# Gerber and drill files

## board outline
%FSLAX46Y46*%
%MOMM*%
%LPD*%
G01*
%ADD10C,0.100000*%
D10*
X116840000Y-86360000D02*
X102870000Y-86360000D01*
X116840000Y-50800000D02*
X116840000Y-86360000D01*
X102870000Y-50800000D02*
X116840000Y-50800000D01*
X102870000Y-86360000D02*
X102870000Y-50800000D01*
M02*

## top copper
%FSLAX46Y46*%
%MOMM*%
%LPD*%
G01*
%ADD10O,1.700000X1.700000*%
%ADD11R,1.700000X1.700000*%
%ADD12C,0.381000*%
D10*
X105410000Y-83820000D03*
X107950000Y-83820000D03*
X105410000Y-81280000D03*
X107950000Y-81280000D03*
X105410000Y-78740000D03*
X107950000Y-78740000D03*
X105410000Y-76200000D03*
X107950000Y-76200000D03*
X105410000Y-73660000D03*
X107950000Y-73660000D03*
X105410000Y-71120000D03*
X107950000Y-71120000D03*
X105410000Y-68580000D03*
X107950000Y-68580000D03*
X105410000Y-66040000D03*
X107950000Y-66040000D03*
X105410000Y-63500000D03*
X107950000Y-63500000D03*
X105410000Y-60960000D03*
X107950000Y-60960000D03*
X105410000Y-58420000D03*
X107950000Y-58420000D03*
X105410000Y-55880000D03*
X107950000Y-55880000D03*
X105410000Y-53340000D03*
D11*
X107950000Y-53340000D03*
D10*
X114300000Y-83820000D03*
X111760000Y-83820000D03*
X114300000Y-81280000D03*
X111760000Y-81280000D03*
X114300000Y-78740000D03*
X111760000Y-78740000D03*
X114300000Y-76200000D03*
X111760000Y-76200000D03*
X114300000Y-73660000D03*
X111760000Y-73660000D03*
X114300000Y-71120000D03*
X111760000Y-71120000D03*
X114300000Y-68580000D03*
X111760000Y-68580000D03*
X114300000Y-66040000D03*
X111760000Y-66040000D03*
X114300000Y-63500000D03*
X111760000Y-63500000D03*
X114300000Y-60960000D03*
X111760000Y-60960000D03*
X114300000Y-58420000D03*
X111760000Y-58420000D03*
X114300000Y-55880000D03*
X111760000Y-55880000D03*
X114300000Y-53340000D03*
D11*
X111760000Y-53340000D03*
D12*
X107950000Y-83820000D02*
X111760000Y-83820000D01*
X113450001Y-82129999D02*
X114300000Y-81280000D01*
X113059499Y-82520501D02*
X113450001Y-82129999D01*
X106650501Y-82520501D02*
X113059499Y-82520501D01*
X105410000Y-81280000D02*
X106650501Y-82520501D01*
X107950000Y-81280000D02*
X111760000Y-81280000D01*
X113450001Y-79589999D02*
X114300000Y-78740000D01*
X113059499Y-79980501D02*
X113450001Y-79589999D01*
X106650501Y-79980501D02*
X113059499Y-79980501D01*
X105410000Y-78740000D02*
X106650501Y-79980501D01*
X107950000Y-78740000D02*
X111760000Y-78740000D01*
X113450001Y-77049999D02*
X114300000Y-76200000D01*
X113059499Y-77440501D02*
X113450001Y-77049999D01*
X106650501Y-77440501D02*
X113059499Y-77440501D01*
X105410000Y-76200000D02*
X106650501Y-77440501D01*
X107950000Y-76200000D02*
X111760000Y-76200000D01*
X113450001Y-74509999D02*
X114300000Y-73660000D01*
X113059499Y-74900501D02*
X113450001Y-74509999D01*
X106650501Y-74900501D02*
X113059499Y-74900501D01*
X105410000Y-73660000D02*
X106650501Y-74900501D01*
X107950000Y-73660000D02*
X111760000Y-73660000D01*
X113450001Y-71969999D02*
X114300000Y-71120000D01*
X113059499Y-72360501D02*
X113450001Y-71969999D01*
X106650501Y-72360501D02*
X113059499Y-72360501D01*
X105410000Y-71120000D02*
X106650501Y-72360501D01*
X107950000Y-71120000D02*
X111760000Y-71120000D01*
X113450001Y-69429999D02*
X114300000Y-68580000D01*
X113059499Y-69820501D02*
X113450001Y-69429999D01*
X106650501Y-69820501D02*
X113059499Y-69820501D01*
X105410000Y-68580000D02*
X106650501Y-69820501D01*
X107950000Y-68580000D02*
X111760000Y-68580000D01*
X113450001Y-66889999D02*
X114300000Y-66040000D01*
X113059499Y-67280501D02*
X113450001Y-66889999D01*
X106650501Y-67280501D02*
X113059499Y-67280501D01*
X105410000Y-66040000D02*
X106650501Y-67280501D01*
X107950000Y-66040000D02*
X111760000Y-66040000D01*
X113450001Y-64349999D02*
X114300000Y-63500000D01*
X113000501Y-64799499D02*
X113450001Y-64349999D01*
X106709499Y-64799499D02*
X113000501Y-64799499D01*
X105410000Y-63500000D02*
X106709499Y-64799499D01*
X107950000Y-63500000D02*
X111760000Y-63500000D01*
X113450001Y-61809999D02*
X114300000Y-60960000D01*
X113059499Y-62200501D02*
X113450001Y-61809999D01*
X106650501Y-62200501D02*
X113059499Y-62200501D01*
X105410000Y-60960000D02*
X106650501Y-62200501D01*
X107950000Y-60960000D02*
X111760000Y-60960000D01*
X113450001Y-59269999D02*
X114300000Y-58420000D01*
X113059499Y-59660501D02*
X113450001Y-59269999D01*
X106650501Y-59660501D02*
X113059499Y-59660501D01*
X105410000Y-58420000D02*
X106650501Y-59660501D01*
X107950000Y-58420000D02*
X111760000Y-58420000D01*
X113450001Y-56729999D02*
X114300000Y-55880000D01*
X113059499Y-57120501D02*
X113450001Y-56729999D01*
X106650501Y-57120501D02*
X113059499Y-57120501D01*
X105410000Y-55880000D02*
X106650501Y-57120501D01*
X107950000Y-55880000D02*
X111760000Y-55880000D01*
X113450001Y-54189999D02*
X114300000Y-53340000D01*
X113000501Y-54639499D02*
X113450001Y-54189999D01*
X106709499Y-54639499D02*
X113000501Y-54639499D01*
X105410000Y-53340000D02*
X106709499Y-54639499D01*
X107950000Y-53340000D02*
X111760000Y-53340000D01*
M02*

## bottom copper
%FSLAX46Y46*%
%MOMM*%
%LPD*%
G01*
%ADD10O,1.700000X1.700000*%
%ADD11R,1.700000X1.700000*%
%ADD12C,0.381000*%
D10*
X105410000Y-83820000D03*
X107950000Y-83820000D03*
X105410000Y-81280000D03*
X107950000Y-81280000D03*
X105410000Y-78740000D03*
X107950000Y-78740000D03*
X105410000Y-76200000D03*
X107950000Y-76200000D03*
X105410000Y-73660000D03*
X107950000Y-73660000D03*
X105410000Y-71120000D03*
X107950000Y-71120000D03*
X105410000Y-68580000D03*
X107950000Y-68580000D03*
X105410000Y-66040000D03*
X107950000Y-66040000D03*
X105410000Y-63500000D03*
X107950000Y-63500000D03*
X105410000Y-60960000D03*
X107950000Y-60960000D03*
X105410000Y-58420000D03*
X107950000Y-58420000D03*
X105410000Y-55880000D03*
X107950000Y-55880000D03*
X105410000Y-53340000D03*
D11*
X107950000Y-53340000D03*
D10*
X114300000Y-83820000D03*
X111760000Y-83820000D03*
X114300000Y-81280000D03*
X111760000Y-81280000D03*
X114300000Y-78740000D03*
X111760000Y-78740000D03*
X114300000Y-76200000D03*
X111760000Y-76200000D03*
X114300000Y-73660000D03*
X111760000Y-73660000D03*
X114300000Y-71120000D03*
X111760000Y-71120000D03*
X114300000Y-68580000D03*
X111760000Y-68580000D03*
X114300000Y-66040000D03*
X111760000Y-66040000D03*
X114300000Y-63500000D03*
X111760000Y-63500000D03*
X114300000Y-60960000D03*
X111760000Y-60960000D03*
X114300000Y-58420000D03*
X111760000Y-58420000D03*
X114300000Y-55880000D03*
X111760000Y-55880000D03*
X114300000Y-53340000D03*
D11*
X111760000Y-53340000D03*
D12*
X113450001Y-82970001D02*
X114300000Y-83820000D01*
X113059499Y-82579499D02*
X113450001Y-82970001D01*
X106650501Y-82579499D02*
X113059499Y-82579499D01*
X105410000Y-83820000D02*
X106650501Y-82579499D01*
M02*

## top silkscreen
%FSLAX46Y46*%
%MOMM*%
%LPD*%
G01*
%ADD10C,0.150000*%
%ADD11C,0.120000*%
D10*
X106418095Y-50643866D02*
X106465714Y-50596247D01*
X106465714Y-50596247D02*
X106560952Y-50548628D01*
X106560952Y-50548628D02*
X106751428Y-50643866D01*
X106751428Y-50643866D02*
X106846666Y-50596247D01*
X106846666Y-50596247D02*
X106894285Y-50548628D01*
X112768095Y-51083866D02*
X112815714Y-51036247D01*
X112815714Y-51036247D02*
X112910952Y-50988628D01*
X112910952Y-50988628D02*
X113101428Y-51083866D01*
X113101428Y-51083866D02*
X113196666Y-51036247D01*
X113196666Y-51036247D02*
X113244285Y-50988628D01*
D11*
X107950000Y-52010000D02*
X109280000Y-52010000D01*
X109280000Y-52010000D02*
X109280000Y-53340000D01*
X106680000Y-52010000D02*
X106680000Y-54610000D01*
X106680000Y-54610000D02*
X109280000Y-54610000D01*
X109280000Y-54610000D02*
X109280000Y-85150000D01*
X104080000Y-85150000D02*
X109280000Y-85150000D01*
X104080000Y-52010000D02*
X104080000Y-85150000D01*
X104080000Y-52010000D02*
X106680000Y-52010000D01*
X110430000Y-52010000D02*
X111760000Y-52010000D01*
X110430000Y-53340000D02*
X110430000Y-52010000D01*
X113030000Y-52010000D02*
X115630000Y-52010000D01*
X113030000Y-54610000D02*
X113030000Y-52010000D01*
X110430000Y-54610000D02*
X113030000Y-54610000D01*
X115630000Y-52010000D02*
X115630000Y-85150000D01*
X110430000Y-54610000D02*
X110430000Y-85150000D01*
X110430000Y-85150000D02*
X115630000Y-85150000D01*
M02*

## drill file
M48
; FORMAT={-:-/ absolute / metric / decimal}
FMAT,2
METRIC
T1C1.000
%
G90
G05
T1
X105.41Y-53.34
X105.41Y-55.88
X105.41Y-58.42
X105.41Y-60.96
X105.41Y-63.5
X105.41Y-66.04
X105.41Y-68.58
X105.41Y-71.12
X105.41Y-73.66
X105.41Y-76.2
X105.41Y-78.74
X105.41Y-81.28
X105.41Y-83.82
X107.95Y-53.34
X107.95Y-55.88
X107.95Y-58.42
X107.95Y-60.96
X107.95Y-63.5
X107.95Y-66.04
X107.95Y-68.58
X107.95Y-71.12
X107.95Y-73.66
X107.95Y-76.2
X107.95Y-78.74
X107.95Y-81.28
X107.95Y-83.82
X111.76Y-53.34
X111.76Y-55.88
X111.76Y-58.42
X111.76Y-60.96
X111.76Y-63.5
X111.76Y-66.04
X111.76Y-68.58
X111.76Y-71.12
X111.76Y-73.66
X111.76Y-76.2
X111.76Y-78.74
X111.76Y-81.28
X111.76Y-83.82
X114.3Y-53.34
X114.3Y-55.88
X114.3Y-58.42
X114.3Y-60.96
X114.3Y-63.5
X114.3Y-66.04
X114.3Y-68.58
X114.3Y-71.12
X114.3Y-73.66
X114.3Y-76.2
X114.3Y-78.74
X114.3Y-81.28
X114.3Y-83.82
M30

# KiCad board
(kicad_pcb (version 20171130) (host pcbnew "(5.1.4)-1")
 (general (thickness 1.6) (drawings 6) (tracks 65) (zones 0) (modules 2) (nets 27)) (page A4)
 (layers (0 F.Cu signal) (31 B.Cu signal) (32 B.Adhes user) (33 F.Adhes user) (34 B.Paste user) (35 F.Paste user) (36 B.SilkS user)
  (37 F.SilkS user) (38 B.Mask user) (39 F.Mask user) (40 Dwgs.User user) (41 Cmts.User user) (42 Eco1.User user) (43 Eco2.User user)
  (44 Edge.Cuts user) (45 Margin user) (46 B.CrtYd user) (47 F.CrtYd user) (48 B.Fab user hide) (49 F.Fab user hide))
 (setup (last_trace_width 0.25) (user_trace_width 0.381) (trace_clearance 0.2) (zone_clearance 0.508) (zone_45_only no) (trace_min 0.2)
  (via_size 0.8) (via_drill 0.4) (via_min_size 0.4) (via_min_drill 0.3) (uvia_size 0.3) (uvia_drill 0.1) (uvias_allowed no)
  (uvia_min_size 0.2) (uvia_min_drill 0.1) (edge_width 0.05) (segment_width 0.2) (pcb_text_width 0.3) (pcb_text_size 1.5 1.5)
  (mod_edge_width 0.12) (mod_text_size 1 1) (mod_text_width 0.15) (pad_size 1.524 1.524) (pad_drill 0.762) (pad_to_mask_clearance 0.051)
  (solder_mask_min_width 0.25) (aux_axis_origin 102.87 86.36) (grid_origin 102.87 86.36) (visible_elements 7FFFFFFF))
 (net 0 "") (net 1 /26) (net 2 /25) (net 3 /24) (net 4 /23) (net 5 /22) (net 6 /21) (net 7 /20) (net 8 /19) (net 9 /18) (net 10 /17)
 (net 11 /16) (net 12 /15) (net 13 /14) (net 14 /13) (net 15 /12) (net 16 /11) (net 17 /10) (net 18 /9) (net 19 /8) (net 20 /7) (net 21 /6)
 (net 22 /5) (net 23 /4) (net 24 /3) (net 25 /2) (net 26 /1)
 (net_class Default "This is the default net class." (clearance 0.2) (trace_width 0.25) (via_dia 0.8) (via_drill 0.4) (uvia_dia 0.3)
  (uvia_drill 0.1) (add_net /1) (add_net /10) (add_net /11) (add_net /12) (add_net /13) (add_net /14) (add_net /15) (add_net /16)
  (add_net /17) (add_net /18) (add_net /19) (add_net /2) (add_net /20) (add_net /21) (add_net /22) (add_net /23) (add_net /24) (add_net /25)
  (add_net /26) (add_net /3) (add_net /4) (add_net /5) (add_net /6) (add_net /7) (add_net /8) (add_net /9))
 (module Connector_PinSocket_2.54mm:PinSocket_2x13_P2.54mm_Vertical (layer F.Cu) (at 107.95 53.34)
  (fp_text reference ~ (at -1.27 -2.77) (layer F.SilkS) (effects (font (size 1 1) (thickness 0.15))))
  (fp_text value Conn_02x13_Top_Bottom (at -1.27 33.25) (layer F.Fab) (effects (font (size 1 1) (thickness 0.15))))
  (fp_line (start 0 -1.33) (end 1.33 -1.33) (layer F.SilkS) (width 0.12))
  (fp_line (start 1.33 -1.33) (end 1.33 0) (layer F.SilkS) (width 0.12))
  (fp_line (start -1.27 -1.33) (end -1.27 1.27) (layer F.SilkS) (width 0.12))
  (fp_line (start -1.27 1.27) (end 1.33 1.27) (layer F.SilkS) (width 0.12))
  (fp_line (start 1.33 1.27) (end 1.33 31.81) (layer F.SilkS) (width 0.12))
  (fp_line (start -3.87 31.81) (end 1.33 31.81) (layer F.SilkS) (width 0.12))
  (fp_line (start -3.87 -1.33) (end -3.87 31.81) (layer F.SilkS) (width 0.12))
  (fp_line (start -3.87 -1.33) (end -1.27 -1.33) (layer F.SilkS) (width 0.12))
  (pad 26 thru_hole oval (at -2.54 30.48) (size 1.7 1.7) (drill 1) (layers *.Cu *.Mask) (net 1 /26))
  (pad 25 thru_hole oval (at 0 30.48) (size 1.7 1.7) (drill 1) (layers *.Cu *.Mask) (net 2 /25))
  (pad 24 thru_hole oval (at -2.54 27.94) (size 1.7 1.7) (drill 1) (layers *.Cu *.Mask) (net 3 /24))
  (pad 23 thru_hole oval (at 0 27.94) (size 1.7 1.7) (drill 1) (layers *.Cu *.Mask) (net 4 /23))
  (pad 22 thru_hole oval (at -2.54 25.4) (size 1.7 1.7) (drill 1) (layers *.Cu *.Mask) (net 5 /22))
  (pad 21 thru_hole oval (at 0 25.4) (size 1.7 1.7) (drill 1) (layers *.Cu *.Mask) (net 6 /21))
  (pad 20 thru_hole oval (at -2.54 22.86) (size 1.7 1.7) (drill 1) (layers *.Cu *.Mask) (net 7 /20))
  (pad 19 thru_hole oval (at 0 22.86) (size 1.7 1.7) (drill 1) (layers *.Cu *.Mask) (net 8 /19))
  (pad 18 thru_hole oval (at -2.54 20.32) (size 1.7 1.7) (drill 1) (layers *.Cu *.Mask) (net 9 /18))
  (pad 17 thru_hole oval (at 0 20.32) (size 1.7 1.7) (drill 1) (layers *.Cu *.Mask) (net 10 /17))
  (pad 16 thru_hole oval (at -2.54 17.78) (size 1.7 1.7) (drill 1) (layers *.Cu *.Mask) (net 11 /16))
  (pad 15 thru_hole oval (at 0 17.78) (size 1.7 1.7) (drill 1) (layers *.Cu *.Mask) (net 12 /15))
  (pad 14 thru_hole oval (at -2.54 15.24) (size 1.7 1.7) (drill 1) (layers *.Cu *.Mask) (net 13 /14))
  (pad 13 thru_hole oval (at 0 15.24) (size 1.7 1.7) (drill 1) (layers *.Cu *.Mask) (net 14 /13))
  (pad 12 thru_hole oval (at -2.54 12.7) (size 1.7 1.7) (drill 1) (layers *.Cu *.Mask) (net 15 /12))
  (pad 11 thru_hole oval (at 0 12.7) (size 1.7 1.7) (drill 1) (layers *.Cu *.Mask) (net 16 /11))
  (pad 10 thru_hole oval (at -2.54 10.16) (size 1.7 1.7) (drill 1) (layers *.Cu *.Mask) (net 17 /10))
  (pad 9 thru_hole oval (at 0 10.16) (size 1.7 1.7) (drill 1) (layers *.Cu *.Mask) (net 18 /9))
  (pad 8 thru_hole oval (at -2.54 7.62) (size 1.7 1.7) (drill 1) (layers *.Cu *.Mask) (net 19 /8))
  (pad 7 thru_hole oval (at 0 7.62) (size 1.7 1.7) (drill 1) (layers *.Cu *.Mask) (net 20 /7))
  (pad 6 thru_hole oval (at -2.54 5.08) (size 1.7 1.7) (drill 1) (layers *.Cu *.Mask) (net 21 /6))
  (pad 5 thru_hole oval (at 0 5.08) (size 1.7 1.7) (drill 1) (layers *.Cu *.Mask) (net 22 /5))
  (pad 4 thru_hole oval (at -2.54 2.54) (size 1.7 1.7) (drill 1) (layers *.Cu *.Mask) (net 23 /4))
  (pad 3 thru_hole oval (at 0 2.54) (size 1.7 1.7) (drill 1) (layers *.Cu *.Mask) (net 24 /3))
  (pad 2 thru_hole oval (at -2.54 0) (size 1.7 1.7) (drill 1) (layers *.Cu *.Mask) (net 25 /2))
  (pad 1 thru_hole rect (at 0 0) (size 1.7 1.7) (drill 1) (layers *.Cu *.Mask) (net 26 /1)))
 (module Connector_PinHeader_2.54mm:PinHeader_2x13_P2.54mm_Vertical (layer F.Cu) (at 111.76 53.34)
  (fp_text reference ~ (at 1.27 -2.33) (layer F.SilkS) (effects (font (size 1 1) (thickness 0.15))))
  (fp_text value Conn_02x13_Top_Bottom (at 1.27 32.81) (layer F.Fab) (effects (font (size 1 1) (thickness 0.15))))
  (fp_line (start -1.33 -1.33) (end 0 -1.33) (layer F.SilkS) (width 0.12))
  (fp_line (start -1.33 0) (end -1.33 -1.33) (layer F.SilkS) (width 0.12))
  (fp_line (start 1.27 -1.33) (end 3.87 -1.33) (layer F.SilkS) (width 0.12))
  (fp_line (start 1.27 1.27) (end 1.27 -1.33) (layer F.SilkS) (width 0.12))
  (fp_line (start -1.33 1.27) (end 1.27 1.27) (layer F.SilkS) (width 0.12))
  (fp_line (start 3.87 -1.33) (end 3.87 31.81) (layer F.SilkS) (width 0.12))
  (fp_line (start -1.33 1.27) (end -1.33 31.81) (layer F.SilkS) (width 0.12))
  (fp_line (start -1.33 31.81) (end 3.87 31.81) (layer F.SilkS) (width 0.12))
  (pad 26 thru_hole oval (at 2.54 30.48) (size 1.7 1.7) (drill 1) (layers *.Cu *.Mask) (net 1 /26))
  (pad 25 thru_hole oval (at 0 30.48) (size 1.7 1.7) (drill 1) (layers *.Cu *.Mask) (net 2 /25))
  (pad 24 thru_hole oval (at 2.54 27.94) (size 1.7 1.7) (drill 1) (layers *.Cu *.Mask) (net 3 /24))
  (pad 23 thru_hole oval (at 0 27.94) (size 1.7 1.7) (drill 1) (layers *.Cu *.Mask) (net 4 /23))
  (pad 22 thru_hole oval (at 2.54 25.4) (size 1.7 1.7) (drill 1) (layers *.Cu *.Mask) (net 5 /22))
  (pad 21 thru_hole oval (at 0 25.4) (size 1.7 1.7) (drill 1) (layers *.Cu *.Mask) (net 6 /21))
  (pad 20 thru_hole oval (at 2.54 22.86) (size 1.7 1.7) (drill 1) (layers *.Cu *.Mask) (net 7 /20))
  (pad 19 thru_hole oval (at 0 22.86) (size 1.7 1.7) (drill 1) (layers *.Cu *.Mask) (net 8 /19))
  (pad 18 thru_hole oval (at 2.54 20.32) (size 1.7 1.7) (drill 1) (layers *.Cu *.Mask) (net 9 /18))
  (pad 17 thru_hole oval (at 0 20.32) (size 1.7 1.7) (drill 1) (layers *.Cu *.Mask) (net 10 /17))
  (pad 16 thru_hole oval (at 2.54 17.78) (size 1.7 1.7) (drill 1) (layers *.Cu *.Mask) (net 11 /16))
  (pad 15 thru_hole oval (at 0 17.78) (size 1.7 1.7) (drill 1) (layers *.Cu *.Mask) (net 12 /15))
  (pad 14 thru_hole oval (at 2.54 15.24) (size 1.7 1.7) (drill 1) (layers *.Cu *.Mask) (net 13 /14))
  (pad 13 thru_hole oval (at 0 15.24) (size 1.7 1.7) (drill 1) (layers *.Cu *.Mask) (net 14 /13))
  (pad 12 thru_hole oval (at 2.54 12.7) (size 1.7 1.7) (drill 1) (layers *.Cu *.Mask) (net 15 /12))
  (pad 11 thru_hole oval (at 0 12.7) (size 1.7 1.7) (drill 1) (layers *.Cu *.Mask) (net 16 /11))
  (pad 10 thru_hole oval (at 2.54 10.16) (size 1.7 1.7) (drill 1) (layers *.Cu *.Mask) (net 17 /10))
  (pad 9 thru_hole oval (at 0 10.16) (size 1.7 1.7) (drill 1) (layers *.Cu *.Mask) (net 18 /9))
  (pad 8 thru_hole oval (at 2.54 7.62) (size 1.7 1.7) (drill 1) (layers *.Cu *.Mask) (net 19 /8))
  (pad 7 thru_hole oval (at 0 7.62) (size 1.7 1.7) (drill 1) (layers *.Cu *.Mask) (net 20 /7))
  (pad 6 thru_hole oval (at 2.54 5.08) (size 1.7 1.7) (drill 1) (layers *.Cu *.Mask) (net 21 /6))
  (pad 5 thru_hole oval (at 0 5.08) (size 1.7 1.7) (drill 1) (layers *.Cu *.Mask) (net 22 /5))
  (pad 4 thru_hole oval (at 2.54 2.54) (size 1.7 1.7) (drill 1) (layers *.Cu *.Mask) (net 23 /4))
  (pad 3 thru_hole oval (at 0 2.54) (size 1.7 1.7) (drill 1) (layers *.Cu *.Mask) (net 24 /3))
  (pad 2 thru_hole oval (at 2.54 0) (size 1.7 1.7) (drill 1) (layers *.Cu *.Mask) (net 25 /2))
  (pad 1 thru_hole rect (at 0 0) (size 1.7 1.7) (drill 1) (layers *.Cu *.Mask) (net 26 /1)))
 (gr_line (start 116.84 86.36) (end 102.87 86.36) (layer Edge.Cuts) (width 0.1))
 (gr_line (start 116.84 50.8) (end 116.84 86.36) (layer Edge.Cuts) (width 0.1))
 (gr_line (start 102.87 50.8) (end 116.84 50.8) (layer Edge.Cuts) (width 0.1))
 (gr_line (start 102.87 86.36) (end 102.87 50.8) (layer Edge.Cuts) (width 0.1))
 (segment (start 113.450001 82.970001) (end 114.3 83.82) (width 0.381) (layer B.Cu) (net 1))
 (segment (start 113.059499 82.579499) (end 113.450001 82.970001) (width 0.381) (layer B.Cu) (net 1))
 (segment (start 106.650501 82.579499) (end 113.059499 82.579499) (width 0.381) (layer B.Cu) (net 1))
 (segment (start 105.41 83.82) (end 106.650501 82.579499) (width 0.381) (layer B.Cu) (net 1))
 (segment (start 107.95 83.82) (end 111.76 83.82) (width 0.381) (layer F.Cu) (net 2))
 (segment (start 113.450001 82.129999) (end 114.3 81.28) (width 0.381) (layer F.Cu) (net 3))
 (segment (start 113.059499 82.520501) (end 113.450001 82.129999) (width 0.381) (layer F.Cu) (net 3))
 (segment (start 106.650501 82.520501) (end 113.059499 82.520501) (width 0.381) (layer F.Cu) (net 3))
 (segment (start 105.41 81.28) (end 106.650501 82.520501) (width 0.381) (layer F.Cu) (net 3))
 (segment (start 107.95 81.28) (end 111.76 81.28) (width 0.381) (layer F.Cu) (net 4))
 (segment (start 113.450001 79.589999) (end 114.3 78.74) (width 0.381) (layer F.Cu) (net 5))
 (segment (start 113.059499 79.980501) (end 113.450001 79.589999) (width 0.381) (layer F.Cu) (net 5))
 (segment (start 106.650501 79.980501) (end 113.059499 79.980501) (width 0.381) (layer F.Cu) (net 5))
 (segment (start 105.41 78.74) (end 106.650501 79.980501) (width 0.381) (layer F.Cu) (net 5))
 (segment (start 107.95 78.74) (end 111.76 78.74) (width 0.381) (layer F.Cu) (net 6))
 (segment (start 113.450001 77.049999) (end 114.3 76.2) (width 0.381) (layer F.Cu) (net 7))
 (segment (start 113.059499 77.440501) (end 113.450001 77.049999) (width 0.381) (layer F.Cu) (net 7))
 (segment (start 106.650501 77.440501) (end 113.059499 77.440501) (width 0.381) (layer F.Cu) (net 7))
 (segment (start 105.41 76.2) (end 106.650501 77.440501) (width 0.381) (layer F.Cu) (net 7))
 (segment (start 107.95 76.2) (end 111.76 76.2) (width 0.381) (layer F.Cu) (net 8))
 (segment (start 113.450001 74.509999) (end 114.3 73.66) (width 0.381) (layer F.Cu) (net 9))
 (segment (start 113.059499 74.900501) (end 113.450001 74.509999) (width 0.381) (layer F.Cu) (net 9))
 (segment (start 106.650501 74.900501) (end 113.059499 74.900501) (width 0.381) (layer F.Cu) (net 9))
 (segment (start 105.41 73.66) (end 106.650501 74.900501) (width 0.381) (layer F.Cu) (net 9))
 (segment (start 107.95 73.66) (end 111.76 73.66) (width 0.381) (layer F.Cu) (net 10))
 (segment (start 113.450001 71.969999) (end 114.3 71.12) (width 0.381) (layer F.Cu) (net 11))
 (segment (start 113.059499 72.360501) (end 113.450001 71.969999) (width 0.381) (layer F.Cu) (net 11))
 (segment (start 106.650501 72.360501) (end 113.059499 72.360501) (width 0.381) (layer F.Cu) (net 11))
 (segment (start 105.41 71.12) (end 106.650501 72.360501) (width 0.381) (layer F.Cu) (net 11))
 (segment (start 107.95 71.12) (end 111.76 71.12) (width 0.381) (layer F.Cu) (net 12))
 (segment (start 113.450001 69.429999) (end 114.3 68.58) (width 0.381) (layer F.Cu) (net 13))
 (segment (start 113.059499 69.820501) (end 113.450001 69.429999) (width 0.381) (layer F.Cu) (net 13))
 (segment (start 106.650501 69.820501) (end 113.059499 69.820501) (width 0.381) (layer F.Cu) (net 13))
 (segment (start 105.41 68.58) (end 106.650501 69.820501) (width 0.381) (layer F.Cu) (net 13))
 (segment (start 107.95 68.58) (end 111.76 68.58) (width 0.381) (layer F.Cu) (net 14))
 (segment (start 113.450001 66.889999) (end 114.3 66.04) (width 0.381) (layer F.Cu) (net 15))
 (segment (start 113.059499 67.280501) (end 113.450001 66.889999) (width 0.381) (layer F.Cu) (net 15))
 (segment (start 106.650501 67.280501) (end 113.059499 67.280501) (width 0.381) (layer F.Cu) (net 15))
 (segment (start 105.41 66.04) (end 106.650501 67.280501) (width 0.381) (layer F.Cu) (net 15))
 (segment (start 107.95 66.04) (end 111.76 66.04) (width 0.381) (layer F.Cu) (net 16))
 (segment (start 113.450001 64.349999) (end 114.3 63.5) (width 0.381) (layer F.Cu) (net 17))
 (segment (start 113.000501 64.799499) (end 113.450001 64.349999) (width 0.381) (layer F.Cu) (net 17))
 (segment (start 106.709499 64.799499) (end 113.000501 64.799499) (width 0.381) (layer F.Cu) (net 17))
 (segment (start 105.41 63.5) (end 106.709499 64.799499) (width 0.381) (layer F.Cu) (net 17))
 (segment (start 107.95 63.5) (end 111.76 63.5) (width 0.381) (layer F.Cu) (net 18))
 (segment (start 113.450001 61.809999) (end 114.3 60.96) (width 0.381) (layer F.Cu) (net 19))
 (segment (start 113.059499 62.200501) (end 113.450001 61.809999) (width 0.381) (layer F.Cu) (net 19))
 (segment (start 106.650501 62.200501) (end 113.059499 62.200501) (width 0.381) (layer F.Cu) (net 19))
 (segment (start 105.41 60.96) (end 106.650501 62.200501) (width 0.381) (layer F.Cu) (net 19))
 (segment (start 107.95 60.96) (end 111.76 60.96) (width 0.381) (layer F.Cu) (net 20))
 (segment (start 113.450001 59.269999) (end 114.3 58.42) (width 0.381) (layer F.Cu) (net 21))
 (segment (start 113.059499 59.660501) (end 113.450001 59.269999) (width 0.381) (layer F.Cu) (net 21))
 (segment (start 106.650501 59.660501) (end 113.059499 59.660501) (width 0.381) (layer F.Cu) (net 21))
 (segment (start 105.41 58.42) (end 106.650501 59.660501) (width 0.381) (layer F.Cu) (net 21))
 (segment (start 107.95 58.42) (end 111.76 58.42) (width 0.381) (layer F.Cu) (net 22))
 (segment (start 113.450001 56.729999) (end 114.3 55.88) (width 0.381) (layer F.Cu) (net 23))
 (segment (start 113.059499 57.120501) (end 113.450001 56.729999) (width 0.381) (layer F.Cu) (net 23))
 (segment (start 106.650501 57.120501) (end 113.059499 57.120501) (width 0.381) (layer F.Cu) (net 23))
 (segment (start 105.41 55.88) (end 106.650501 57.120501) (width 0.381) (layer F.Cu) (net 23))
 (segment (start 107.95 55.88) (end 111.76 55.88) (width 0.381) (layer F.Cu) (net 24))
 (segment (start 113.450001 54.189999) (end 114.3 53.34) (width 0.381) (layer F.Cu) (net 25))
 (segment (start 113.000501 54.639499) (end 113.450001 54.189999) (width 0.381) (layer F.Cu) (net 25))
 (segment (start 106.709499 54.639499) (end 113.000501 54.639499) (width 0.381) (layer F.Cu) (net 25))
 (segment (start 105.41 53.34) (end 106.709499 54.639499) (width 0.381) (layer F.Cu) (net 25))
 (segment (start 107.95 53.34) (end 111.76 53.34) (width 0.381) (layer F.Cu) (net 26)))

